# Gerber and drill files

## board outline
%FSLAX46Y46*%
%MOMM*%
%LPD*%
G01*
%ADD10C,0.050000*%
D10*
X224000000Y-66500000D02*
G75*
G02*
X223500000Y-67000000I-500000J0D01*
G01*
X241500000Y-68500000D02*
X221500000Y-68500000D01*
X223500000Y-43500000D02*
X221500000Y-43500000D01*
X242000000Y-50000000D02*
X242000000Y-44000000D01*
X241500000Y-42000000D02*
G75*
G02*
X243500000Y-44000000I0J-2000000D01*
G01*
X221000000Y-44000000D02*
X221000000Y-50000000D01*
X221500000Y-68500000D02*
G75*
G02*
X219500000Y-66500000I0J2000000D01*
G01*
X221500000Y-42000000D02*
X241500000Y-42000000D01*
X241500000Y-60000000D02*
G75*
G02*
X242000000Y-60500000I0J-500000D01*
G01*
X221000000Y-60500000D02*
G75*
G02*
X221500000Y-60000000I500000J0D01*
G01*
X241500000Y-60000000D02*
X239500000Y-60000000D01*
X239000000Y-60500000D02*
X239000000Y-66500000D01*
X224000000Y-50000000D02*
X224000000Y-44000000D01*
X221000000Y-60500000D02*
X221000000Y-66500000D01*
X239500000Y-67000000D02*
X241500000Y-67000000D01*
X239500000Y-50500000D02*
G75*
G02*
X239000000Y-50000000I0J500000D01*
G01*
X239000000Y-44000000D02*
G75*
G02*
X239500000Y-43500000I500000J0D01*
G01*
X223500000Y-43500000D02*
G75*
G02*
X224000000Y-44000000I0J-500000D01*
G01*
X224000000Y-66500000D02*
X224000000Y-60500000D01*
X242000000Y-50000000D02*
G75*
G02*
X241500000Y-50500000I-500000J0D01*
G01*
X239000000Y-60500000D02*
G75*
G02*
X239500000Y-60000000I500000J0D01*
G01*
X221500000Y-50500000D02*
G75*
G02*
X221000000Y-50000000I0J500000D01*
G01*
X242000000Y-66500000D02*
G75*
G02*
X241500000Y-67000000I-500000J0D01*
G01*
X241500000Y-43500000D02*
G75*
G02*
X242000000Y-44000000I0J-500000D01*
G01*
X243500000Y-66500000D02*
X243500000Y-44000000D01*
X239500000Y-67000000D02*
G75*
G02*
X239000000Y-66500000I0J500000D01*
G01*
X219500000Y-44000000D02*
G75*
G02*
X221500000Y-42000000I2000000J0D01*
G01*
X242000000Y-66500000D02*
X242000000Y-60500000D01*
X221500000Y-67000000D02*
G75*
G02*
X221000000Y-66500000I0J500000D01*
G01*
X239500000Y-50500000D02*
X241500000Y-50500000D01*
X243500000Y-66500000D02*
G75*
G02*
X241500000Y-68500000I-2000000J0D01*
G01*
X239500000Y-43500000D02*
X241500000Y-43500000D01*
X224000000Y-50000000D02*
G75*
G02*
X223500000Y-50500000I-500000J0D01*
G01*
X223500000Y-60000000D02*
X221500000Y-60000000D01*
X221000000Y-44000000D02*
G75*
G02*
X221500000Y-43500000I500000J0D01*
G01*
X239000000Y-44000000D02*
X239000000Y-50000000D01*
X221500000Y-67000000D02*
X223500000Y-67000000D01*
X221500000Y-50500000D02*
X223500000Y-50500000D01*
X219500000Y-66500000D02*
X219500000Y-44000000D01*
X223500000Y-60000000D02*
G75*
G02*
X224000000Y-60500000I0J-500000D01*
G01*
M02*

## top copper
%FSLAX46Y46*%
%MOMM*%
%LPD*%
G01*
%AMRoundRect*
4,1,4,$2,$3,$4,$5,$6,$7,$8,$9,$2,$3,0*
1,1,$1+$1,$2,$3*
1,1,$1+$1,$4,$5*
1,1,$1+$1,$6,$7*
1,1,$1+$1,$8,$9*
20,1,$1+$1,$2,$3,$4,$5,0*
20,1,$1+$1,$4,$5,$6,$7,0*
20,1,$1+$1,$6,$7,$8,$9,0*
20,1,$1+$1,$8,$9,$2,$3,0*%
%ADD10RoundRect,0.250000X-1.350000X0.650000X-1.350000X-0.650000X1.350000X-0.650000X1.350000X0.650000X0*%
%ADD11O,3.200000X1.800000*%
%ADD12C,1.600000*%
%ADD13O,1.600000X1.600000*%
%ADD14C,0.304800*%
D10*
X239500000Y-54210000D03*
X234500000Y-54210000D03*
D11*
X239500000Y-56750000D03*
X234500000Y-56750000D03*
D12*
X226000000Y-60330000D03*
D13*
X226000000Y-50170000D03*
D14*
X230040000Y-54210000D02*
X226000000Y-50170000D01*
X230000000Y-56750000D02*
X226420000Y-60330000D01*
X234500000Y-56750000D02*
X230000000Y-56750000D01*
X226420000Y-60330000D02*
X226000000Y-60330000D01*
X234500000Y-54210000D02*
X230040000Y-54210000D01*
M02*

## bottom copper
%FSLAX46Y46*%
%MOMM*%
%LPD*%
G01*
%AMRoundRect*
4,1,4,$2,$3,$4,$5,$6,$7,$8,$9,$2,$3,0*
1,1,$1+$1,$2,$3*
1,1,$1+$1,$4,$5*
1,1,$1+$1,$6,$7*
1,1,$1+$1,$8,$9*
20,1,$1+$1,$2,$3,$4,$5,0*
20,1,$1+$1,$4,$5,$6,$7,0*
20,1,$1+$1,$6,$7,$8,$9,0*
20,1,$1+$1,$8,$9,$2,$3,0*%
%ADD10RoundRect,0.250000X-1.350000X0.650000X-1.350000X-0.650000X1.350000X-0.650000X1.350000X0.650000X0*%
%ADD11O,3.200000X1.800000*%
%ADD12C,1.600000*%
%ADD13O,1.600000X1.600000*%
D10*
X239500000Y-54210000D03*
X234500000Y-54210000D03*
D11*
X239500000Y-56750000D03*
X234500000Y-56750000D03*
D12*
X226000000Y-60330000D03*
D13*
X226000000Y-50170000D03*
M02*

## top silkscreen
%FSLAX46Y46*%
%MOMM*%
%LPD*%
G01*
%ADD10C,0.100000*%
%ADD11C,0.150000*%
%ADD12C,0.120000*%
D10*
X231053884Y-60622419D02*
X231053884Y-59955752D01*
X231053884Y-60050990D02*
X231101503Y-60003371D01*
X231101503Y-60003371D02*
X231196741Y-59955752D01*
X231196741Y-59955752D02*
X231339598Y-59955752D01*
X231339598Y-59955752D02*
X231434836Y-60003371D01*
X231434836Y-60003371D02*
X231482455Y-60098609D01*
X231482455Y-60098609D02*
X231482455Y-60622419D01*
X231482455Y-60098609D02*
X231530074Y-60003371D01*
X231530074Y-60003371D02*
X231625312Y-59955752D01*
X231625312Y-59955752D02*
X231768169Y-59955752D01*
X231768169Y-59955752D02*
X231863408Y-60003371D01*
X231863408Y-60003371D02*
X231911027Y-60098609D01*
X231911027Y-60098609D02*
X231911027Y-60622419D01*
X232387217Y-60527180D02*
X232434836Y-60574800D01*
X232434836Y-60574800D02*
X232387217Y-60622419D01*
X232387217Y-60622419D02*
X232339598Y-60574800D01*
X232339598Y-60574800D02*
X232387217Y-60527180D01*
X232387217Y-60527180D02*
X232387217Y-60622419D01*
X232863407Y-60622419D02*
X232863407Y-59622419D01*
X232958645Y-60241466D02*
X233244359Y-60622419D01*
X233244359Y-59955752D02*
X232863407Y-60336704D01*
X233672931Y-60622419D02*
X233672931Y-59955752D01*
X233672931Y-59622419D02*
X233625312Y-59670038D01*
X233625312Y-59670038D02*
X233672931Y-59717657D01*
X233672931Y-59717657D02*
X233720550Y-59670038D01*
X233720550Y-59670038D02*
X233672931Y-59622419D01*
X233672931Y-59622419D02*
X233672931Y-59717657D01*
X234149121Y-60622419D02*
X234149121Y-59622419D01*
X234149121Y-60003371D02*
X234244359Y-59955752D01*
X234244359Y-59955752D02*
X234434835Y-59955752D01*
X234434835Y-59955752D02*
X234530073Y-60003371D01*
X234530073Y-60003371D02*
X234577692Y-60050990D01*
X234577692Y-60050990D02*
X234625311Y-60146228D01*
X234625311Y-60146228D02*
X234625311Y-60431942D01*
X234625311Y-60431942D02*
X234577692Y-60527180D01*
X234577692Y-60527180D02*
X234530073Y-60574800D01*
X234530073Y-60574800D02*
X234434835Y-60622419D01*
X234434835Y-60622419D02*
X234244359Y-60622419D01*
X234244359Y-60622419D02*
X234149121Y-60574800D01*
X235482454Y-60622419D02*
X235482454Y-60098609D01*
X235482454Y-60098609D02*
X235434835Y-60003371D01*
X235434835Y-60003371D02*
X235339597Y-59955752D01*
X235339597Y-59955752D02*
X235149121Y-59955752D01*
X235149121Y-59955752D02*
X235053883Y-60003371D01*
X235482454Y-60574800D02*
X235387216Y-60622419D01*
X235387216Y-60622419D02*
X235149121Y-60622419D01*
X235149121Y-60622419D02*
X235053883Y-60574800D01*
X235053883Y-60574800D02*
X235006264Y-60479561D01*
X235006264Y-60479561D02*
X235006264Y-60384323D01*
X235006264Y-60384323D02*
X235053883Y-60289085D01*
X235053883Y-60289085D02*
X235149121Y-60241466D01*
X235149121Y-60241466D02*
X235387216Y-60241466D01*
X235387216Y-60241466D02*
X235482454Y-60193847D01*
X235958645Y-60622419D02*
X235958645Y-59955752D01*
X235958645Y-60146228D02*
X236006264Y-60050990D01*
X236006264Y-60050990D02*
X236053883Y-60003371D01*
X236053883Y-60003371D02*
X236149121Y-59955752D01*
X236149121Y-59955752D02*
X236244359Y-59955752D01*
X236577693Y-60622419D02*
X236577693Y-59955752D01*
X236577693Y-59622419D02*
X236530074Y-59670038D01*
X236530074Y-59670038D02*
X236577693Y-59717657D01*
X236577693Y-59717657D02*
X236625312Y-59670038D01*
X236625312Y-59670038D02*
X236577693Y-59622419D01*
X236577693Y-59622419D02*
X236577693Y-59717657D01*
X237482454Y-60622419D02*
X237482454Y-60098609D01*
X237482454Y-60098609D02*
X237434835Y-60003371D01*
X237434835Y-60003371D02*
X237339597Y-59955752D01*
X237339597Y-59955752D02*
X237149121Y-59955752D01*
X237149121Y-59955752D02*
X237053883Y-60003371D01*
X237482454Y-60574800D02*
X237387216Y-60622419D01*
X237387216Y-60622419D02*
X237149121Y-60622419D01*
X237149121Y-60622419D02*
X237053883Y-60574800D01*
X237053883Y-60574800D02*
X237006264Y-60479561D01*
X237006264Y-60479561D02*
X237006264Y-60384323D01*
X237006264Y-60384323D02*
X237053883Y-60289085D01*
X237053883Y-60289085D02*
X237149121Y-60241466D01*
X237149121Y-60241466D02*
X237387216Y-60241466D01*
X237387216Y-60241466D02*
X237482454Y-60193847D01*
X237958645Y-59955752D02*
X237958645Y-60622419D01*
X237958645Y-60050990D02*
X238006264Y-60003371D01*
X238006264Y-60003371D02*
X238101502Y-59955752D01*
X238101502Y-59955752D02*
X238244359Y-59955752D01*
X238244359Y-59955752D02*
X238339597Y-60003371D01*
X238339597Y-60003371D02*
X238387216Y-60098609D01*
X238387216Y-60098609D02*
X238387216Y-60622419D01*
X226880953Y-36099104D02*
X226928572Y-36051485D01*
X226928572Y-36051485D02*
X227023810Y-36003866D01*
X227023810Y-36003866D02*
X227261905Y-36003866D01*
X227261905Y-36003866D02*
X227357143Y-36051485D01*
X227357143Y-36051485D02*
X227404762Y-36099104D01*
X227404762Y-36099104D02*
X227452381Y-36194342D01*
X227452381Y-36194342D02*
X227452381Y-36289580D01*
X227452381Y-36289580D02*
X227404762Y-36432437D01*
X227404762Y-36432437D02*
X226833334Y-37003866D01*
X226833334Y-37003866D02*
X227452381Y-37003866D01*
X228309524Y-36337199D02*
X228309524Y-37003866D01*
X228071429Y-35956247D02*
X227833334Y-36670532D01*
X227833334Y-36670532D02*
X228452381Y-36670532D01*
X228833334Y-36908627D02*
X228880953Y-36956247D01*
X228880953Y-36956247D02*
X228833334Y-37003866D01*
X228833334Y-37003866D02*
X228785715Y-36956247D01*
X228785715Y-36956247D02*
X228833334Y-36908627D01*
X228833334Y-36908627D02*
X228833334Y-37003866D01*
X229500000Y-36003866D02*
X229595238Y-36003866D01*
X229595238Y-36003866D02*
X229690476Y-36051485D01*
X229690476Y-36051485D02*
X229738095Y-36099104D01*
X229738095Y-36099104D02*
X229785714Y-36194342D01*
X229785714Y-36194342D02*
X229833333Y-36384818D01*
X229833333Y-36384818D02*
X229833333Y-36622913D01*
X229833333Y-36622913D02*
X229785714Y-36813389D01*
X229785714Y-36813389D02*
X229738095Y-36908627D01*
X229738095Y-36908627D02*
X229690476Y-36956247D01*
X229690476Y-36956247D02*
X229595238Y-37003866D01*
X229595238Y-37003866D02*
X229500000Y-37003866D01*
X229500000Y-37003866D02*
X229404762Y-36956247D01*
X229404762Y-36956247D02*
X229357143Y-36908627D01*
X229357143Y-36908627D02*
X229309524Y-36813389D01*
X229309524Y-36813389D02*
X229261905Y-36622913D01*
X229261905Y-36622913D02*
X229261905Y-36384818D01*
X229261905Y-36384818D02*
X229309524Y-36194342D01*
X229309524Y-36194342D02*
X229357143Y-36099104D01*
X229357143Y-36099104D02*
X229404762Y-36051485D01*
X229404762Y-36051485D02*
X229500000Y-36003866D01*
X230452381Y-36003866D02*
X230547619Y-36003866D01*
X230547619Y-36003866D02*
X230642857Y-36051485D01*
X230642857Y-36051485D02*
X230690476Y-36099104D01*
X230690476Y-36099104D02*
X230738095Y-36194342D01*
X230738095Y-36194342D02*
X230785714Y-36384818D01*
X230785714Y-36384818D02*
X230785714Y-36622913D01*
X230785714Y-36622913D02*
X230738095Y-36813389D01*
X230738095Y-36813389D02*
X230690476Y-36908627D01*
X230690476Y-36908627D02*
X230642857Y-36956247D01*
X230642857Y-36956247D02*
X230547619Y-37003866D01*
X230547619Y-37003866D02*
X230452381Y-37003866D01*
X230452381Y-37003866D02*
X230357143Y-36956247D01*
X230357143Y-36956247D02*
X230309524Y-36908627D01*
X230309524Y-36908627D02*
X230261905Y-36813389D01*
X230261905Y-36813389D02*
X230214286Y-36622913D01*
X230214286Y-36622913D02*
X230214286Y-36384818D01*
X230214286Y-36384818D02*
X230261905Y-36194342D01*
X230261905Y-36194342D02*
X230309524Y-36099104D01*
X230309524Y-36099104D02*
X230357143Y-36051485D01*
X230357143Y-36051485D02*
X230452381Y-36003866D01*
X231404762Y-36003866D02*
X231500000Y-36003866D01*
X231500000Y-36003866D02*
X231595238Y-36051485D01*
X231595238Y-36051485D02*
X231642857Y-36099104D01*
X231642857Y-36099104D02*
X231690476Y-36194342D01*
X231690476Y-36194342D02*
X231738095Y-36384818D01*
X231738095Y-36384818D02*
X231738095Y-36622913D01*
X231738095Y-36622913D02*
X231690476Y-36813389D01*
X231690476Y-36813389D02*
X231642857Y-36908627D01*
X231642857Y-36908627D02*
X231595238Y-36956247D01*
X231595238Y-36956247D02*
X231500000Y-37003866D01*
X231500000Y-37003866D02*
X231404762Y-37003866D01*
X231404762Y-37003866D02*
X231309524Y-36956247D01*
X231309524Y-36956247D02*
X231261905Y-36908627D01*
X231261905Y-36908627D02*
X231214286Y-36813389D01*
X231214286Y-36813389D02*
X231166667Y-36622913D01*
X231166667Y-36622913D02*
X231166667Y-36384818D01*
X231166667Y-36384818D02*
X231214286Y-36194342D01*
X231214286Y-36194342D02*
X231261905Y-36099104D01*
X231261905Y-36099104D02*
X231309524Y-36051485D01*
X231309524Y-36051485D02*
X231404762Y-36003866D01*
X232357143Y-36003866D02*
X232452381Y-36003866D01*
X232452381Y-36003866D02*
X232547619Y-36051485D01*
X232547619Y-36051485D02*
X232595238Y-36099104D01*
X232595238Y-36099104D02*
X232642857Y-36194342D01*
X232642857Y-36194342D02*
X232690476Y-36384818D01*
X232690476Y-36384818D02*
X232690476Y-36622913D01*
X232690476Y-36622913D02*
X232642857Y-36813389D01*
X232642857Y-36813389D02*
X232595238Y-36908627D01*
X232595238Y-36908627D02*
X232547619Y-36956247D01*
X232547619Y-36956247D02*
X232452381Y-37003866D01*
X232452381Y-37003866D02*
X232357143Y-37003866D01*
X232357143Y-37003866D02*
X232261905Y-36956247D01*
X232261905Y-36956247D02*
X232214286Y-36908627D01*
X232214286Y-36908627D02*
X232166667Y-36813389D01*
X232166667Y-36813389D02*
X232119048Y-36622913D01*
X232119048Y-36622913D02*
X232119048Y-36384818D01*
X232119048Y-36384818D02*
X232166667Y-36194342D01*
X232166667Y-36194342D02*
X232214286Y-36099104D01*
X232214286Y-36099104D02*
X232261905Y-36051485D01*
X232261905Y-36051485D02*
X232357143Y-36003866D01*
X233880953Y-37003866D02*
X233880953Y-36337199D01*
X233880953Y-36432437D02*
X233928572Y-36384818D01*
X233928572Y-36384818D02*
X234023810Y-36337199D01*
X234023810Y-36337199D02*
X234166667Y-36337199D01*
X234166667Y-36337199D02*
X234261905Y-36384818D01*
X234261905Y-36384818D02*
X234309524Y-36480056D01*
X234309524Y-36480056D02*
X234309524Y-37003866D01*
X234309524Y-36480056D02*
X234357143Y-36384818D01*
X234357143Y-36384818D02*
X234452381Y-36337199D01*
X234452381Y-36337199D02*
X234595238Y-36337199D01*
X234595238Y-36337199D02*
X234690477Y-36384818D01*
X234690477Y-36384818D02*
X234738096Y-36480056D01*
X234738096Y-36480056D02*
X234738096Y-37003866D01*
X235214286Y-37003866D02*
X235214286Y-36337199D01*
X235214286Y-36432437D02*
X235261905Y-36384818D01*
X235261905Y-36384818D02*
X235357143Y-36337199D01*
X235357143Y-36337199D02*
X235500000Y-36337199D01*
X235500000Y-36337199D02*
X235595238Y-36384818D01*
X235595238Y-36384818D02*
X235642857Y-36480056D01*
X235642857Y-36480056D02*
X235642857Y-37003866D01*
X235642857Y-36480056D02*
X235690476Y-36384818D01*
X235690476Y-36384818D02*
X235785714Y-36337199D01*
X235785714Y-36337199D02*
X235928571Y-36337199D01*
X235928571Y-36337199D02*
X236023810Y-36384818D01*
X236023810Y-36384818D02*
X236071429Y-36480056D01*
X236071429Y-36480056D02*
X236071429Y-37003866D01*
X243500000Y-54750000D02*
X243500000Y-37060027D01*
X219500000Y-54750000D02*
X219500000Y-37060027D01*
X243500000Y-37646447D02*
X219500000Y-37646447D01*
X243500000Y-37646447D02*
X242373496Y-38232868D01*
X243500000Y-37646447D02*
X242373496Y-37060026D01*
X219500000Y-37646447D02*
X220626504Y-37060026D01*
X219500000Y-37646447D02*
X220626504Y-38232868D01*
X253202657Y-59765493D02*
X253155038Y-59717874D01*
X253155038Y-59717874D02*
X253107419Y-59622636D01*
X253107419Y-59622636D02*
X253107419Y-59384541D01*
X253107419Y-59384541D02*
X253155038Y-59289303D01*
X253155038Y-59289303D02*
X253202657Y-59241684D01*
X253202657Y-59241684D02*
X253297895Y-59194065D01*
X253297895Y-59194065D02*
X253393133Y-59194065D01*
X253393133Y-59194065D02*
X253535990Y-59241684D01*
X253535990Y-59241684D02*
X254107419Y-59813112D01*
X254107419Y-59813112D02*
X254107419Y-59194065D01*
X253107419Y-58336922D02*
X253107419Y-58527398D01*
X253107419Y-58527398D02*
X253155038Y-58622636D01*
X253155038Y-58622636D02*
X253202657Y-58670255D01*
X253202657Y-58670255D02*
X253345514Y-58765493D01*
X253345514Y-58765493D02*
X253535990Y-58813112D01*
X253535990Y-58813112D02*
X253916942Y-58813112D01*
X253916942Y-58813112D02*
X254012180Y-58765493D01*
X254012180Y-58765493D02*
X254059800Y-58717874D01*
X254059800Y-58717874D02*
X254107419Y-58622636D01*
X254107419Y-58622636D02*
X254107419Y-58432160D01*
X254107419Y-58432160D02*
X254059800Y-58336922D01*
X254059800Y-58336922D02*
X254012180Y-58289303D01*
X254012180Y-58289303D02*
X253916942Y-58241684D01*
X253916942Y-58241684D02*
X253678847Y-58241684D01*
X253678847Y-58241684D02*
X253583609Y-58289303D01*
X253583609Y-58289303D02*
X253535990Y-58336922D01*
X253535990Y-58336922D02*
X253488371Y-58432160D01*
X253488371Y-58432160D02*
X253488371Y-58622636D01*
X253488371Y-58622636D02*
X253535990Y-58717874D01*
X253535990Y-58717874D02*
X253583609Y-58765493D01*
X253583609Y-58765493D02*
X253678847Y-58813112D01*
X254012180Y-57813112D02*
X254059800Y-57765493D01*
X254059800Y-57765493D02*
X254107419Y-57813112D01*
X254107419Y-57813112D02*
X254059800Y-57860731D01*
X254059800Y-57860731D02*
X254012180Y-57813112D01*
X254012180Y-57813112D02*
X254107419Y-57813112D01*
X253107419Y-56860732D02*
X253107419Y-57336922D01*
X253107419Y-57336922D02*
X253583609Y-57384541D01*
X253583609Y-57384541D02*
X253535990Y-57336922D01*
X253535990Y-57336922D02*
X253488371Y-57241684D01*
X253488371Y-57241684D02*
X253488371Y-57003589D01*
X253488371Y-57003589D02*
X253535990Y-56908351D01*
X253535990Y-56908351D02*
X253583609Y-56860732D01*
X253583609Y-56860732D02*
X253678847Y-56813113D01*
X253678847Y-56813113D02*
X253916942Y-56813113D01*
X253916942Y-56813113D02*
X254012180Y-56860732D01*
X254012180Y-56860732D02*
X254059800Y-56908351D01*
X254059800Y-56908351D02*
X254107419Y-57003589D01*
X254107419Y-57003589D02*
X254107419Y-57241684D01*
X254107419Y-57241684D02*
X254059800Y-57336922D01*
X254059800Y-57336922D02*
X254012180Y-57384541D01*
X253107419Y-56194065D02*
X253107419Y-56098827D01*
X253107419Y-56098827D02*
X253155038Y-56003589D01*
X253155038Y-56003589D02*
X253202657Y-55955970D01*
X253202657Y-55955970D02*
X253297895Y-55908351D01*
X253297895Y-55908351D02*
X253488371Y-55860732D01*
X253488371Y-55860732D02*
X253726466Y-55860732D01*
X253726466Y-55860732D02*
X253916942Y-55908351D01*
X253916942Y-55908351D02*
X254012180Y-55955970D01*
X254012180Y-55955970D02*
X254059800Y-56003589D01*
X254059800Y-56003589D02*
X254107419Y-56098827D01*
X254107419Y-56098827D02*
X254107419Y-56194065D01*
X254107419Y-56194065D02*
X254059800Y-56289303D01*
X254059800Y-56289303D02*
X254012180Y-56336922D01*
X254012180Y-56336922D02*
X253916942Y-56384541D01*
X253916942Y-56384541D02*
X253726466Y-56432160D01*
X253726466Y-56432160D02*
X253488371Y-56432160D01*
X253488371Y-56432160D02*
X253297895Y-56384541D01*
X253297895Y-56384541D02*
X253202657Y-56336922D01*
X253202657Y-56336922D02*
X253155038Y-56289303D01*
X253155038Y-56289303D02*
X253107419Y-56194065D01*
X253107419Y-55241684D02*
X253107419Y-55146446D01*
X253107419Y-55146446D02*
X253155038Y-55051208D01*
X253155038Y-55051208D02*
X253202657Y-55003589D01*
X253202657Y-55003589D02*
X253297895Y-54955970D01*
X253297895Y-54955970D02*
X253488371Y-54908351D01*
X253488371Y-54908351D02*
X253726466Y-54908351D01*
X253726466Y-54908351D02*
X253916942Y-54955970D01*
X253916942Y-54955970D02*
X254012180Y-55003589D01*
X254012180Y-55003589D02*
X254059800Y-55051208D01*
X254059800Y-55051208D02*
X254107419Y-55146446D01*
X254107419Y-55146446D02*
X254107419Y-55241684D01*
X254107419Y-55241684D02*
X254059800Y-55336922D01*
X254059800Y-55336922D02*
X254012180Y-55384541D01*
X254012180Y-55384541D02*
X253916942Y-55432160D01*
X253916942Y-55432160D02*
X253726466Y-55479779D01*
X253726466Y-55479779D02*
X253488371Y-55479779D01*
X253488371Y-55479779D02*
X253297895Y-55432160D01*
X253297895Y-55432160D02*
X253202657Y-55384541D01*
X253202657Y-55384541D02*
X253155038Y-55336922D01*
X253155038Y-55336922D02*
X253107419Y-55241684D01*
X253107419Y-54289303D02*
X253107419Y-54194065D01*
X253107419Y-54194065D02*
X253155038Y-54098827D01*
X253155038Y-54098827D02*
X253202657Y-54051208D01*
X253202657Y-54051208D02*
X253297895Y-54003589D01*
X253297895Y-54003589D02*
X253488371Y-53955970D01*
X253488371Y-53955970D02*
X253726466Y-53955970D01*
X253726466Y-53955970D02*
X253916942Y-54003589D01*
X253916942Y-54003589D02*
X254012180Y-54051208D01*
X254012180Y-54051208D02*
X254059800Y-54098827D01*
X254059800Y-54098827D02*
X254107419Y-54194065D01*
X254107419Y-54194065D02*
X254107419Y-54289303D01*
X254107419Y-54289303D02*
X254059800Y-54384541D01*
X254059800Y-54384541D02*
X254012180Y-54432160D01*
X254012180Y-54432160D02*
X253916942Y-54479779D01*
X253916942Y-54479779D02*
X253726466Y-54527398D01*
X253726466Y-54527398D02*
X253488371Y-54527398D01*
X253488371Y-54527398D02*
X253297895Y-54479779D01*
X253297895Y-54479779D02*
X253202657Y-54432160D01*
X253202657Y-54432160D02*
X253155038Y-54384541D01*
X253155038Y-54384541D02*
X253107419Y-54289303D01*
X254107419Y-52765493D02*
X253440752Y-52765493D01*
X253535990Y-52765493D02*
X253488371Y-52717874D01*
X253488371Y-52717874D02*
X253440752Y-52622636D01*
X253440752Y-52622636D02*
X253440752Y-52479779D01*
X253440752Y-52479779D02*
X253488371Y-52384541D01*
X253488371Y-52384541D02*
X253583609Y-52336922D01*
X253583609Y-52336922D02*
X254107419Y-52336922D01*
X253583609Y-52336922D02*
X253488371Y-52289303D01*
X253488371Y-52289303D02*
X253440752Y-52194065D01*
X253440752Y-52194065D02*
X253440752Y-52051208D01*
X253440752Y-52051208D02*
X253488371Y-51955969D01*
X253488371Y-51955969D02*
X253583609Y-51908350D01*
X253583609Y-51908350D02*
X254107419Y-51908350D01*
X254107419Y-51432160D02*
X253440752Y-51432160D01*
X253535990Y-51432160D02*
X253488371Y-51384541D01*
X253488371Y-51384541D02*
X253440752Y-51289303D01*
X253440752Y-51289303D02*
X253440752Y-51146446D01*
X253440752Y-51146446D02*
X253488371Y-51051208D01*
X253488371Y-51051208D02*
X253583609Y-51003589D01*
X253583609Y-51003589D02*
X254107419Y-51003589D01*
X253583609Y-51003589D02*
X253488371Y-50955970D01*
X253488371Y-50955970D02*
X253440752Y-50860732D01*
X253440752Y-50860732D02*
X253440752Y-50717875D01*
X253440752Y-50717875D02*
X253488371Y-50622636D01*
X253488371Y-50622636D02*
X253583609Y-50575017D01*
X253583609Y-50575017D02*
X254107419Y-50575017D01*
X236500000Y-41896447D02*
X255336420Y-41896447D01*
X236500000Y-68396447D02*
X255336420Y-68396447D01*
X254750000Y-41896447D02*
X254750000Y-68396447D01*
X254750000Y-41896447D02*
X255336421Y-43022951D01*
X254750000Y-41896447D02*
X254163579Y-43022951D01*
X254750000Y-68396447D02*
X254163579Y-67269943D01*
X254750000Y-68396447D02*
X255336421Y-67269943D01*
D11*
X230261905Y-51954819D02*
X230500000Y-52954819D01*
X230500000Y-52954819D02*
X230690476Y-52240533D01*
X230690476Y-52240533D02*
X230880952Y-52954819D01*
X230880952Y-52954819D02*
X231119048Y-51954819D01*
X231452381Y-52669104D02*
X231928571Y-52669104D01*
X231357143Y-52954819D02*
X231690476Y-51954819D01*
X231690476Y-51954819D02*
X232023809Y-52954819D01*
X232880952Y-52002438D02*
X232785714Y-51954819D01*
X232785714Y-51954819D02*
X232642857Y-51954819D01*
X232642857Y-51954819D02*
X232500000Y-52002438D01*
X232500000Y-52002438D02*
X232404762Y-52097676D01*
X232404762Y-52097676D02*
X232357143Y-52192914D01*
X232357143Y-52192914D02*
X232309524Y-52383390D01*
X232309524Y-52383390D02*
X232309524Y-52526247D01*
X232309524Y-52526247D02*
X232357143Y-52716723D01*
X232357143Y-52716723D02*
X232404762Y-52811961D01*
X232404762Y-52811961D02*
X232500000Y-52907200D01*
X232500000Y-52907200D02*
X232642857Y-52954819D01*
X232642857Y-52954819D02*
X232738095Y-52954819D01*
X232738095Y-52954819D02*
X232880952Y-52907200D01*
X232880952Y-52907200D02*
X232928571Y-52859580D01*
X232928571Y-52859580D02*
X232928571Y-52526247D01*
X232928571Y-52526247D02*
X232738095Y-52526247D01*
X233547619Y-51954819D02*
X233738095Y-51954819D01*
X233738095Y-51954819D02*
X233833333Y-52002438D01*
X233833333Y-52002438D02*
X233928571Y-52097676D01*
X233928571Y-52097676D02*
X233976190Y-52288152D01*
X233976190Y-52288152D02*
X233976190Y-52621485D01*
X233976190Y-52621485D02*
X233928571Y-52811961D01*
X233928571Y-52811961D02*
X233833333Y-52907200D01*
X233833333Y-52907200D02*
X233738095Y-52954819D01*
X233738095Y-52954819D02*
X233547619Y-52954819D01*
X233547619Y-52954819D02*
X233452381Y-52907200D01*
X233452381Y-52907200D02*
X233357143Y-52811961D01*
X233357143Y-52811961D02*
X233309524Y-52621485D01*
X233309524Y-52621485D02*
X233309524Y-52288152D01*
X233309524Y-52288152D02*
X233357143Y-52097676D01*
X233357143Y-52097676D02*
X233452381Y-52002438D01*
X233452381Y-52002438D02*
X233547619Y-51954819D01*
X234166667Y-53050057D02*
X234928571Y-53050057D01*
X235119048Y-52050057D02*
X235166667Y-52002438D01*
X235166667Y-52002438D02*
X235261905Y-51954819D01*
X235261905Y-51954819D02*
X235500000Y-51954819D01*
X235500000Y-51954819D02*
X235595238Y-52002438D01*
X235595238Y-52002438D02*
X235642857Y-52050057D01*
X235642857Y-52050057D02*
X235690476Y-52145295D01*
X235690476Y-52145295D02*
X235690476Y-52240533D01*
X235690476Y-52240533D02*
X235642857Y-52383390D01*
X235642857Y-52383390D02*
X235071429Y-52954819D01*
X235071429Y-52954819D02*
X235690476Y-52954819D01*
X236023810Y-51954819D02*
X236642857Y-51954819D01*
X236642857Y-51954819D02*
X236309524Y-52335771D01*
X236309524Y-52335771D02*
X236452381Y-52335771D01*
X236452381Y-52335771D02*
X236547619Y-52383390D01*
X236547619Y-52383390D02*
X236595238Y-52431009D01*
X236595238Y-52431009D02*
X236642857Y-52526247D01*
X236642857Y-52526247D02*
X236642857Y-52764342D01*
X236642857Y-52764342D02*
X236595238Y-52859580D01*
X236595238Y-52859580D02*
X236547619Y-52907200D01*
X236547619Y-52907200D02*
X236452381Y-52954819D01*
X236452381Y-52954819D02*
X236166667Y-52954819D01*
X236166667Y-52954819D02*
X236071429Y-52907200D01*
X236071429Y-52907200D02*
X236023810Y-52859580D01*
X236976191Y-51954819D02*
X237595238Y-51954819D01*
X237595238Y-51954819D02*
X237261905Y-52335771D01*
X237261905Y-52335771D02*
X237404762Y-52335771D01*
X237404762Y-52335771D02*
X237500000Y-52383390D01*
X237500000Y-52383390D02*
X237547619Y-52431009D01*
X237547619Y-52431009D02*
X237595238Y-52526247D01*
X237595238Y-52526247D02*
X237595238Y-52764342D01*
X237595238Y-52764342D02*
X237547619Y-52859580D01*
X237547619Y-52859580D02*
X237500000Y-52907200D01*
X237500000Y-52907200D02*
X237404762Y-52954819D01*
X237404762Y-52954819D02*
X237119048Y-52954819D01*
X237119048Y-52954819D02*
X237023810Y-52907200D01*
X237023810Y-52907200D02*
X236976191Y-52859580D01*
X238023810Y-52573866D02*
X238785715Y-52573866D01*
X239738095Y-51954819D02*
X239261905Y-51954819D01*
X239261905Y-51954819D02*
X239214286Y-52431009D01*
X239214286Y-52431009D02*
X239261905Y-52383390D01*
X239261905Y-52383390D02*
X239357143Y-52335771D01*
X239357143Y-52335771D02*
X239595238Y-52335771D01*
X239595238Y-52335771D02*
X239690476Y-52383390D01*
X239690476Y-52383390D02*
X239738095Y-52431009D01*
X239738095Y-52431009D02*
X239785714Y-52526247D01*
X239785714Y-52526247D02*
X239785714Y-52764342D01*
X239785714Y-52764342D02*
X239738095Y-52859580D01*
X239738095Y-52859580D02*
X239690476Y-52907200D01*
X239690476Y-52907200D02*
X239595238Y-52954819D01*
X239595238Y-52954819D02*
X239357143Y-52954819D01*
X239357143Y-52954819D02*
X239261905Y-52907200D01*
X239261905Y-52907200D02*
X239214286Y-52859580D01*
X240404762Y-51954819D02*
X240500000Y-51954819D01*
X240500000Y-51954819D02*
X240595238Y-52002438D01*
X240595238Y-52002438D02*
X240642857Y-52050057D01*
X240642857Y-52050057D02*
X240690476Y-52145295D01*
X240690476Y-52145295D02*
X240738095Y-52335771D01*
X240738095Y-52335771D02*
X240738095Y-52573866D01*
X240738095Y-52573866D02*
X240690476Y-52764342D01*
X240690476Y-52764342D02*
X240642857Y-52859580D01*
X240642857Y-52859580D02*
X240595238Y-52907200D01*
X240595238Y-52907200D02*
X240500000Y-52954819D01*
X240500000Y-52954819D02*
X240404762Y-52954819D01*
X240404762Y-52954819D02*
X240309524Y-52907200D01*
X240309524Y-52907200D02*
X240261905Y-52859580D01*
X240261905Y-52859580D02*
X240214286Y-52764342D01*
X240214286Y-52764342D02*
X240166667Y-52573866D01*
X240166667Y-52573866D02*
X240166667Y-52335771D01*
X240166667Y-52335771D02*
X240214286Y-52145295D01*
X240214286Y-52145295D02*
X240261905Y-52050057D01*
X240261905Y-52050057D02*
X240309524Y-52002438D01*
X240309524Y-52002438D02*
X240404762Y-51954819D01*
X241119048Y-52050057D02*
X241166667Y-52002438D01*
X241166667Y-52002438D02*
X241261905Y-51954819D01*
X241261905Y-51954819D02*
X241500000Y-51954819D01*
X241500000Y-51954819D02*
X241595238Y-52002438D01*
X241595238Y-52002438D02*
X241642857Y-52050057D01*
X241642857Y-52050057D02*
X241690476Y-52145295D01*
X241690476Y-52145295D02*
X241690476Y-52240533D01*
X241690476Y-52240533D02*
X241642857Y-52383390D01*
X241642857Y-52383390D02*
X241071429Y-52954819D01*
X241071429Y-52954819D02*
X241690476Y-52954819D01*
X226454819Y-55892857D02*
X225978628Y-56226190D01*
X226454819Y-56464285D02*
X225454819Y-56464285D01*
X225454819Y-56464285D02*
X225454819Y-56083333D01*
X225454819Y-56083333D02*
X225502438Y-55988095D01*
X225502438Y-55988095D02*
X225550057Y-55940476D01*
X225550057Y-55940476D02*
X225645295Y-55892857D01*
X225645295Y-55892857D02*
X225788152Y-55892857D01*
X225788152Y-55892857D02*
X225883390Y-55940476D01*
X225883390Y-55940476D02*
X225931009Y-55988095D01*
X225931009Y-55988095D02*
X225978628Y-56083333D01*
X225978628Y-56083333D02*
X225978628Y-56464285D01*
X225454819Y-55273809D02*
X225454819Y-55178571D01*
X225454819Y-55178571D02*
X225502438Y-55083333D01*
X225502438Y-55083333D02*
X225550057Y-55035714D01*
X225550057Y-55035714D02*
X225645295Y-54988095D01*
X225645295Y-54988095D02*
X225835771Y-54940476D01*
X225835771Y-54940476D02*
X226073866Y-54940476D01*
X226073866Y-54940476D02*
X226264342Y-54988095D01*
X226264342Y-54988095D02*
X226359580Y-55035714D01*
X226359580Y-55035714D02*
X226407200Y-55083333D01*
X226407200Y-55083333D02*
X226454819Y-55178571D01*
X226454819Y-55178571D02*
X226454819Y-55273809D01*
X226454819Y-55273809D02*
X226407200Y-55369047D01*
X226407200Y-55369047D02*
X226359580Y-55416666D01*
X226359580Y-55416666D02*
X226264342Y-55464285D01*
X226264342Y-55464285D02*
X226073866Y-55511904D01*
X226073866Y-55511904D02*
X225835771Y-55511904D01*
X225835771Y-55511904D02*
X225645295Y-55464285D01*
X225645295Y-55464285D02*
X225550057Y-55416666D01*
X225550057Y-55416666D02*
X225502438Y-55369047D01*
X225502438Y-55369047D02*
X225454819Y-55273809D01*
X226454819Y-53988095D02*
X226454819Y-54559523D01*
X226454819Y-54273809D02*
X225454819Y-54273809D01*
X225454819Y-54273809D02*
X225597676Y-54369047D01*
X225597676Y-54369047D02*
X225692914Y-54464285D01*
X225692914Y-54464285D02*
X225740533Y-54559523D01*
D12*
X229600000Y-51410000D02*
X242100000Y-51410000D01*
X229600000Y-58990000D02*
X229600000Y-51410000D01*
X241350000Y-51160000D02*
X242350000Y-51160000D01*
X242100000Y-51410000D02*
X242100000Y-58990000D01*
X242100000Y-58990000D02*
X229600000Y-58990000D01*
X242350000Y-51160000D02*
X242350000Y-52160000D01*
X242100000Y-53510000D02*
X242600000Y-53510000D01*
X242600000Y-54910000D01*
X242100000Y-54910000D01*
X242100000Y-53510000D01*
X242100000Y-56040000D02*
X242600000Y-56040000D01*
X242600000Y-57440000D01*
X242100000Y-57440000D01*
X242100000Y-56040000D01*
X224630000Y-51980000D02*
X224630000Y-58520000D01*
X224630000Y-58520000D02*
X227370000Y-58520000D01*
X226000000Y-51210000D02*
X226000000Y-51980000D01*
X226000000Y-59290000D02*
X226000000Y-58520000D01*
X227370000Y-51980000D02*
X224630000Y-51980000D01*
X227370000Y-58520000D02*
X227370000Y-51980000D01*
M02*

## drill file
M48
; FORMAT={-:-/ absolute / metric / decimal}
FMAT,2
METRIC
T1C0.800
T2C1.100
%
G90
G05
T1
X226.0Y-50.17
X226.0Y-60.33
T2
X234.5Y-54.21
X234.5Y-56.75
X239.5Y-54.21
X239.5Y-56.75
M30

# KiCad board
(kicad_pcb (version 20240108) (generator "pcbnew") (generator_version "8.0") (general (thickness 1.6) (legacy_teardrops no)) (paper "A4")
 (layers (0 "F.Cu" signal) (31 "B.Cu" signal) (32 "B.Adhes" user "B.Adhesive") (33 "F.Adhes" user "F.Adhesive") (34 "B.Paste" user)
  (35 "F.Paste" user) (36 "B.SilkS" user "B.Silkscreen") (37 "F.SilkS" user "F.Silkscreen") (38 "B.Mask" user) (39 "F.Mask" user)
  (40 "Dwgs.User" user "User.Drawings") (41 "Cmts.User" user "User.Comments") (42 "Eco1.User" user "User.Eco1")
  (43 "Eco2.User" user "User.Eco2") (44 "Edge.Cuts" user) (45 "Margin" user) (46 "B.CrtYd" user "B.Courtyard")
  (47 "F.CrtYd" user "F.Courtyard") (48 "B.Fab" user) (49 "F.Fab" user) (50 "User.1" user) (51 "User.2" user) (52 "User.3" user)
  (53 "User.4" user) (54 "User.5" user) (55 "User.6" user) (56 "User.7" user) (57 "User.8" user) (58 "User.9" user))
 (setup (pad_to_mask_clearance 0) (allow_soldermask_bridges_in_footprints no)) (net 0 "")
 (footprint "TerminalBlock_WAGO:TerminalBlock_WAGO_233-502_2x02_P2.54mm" (layer "F.Cu") (at 239.5 54.21 -90)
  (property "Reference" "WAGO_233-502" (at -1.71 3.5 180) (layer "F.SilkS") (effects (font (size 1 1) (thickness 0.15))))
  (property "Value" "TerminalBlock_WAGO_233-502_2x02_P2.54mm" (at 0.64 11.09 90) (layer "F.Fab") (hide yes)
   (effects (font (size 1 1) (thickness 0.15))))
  (fp_line (start -2.8 9.9) (end -2.8 -2.6) (stroke (width 0.12) (type solid)) (layer "F.SilkS"))
  (fp_line (start 4.78 9.9) (end -2.8 9.9) (stroke (width 0.12) (type solid)) (layer "F.SilkS"))
  (fp_line (start -3.05 -1.85) (end -3.05 -2.85) (stroke (width 0.12) (type default)) (layer "F.SilkS"))
  (fp_line (start -2.8 -2.6) (end 4.78 -2.6) (stroke (width 0.12) (type solid)) (layer "F.SilkS"))
  (fp_line (start 4.78 -2.6) (end 4.78 9.9) (stroke (width 0.12) (type solid)) (layer "F.SilkS"))
  (fp_line (start -3.05 -2.85) (end -2.05 -2.85) (stroke (width 0.12) (type default)) (layer "F.SilkS"))
  (fp_rect (start -0.7 -3.1) (end 0.7 -2.6) (stroke (width 0.12) (type default)) (fill none) (layer "F.SilkS"))
  (fp_rect (start 1.83 -3.1) (end 3.23 -2.6) (stroke (width 0.12) (type default)) (fill none) (layer "F.SilkS"))
  (pad "1" thru_hole roundrect (at 0 0 270) (size 1.8 3.2) (drill 1.1) (layers "*.Cu" "*.Mask") (remove_unused_layers no)
   (roundrect_rratio 0.1388888889))
  (pad "1" thru_hole roundrect (at 0 5 270) (size 1.8 3.2) (drill 1.1) (layers "*.Cu" "*.Mask") (remove_unused_layers no)
   (roundrect_rratio 0.1388888889))
  (pad "2" thru_hole oval (at 2.54 0 270) (size 1.8 3.2) (drill 1.1) (layers "*.Cu" "*.Mask") (remove_unused_layers no))
  (pad "2" thru_hole oval (at 2.54 5 270) (size 1.8 3.2) (drill 1.1) (layers "*.Cu" "*.Mask") (remove_unused_layers no)))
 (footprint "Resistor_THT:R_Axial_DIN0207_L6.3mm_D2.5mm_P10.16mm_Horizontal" (layer "F.Cu") (at 226 60.33 90)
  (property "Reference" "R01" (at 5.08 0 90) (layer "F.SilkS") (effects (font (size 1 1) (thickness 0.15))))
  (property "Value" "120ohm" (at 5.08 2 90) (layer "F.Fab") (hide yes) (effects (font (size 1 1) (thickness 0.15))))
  (fp_line (start 8.35 -1.37) (end 1.81 -1.37) (stroke (width 0.12) (type solid)) (layer "F.SilkS"))
  (fp_line (start 1.81 -1.37) (end 1.81 1.37) (stroke (width 0.12) (type solid)) (layer "F.SilkS"))
  (fp_line (start 9.12 0) (end 8.35 0) (stroke (width 0.12) (type solid)) (layer "F.SilkS"))
  (fp_line (start 1.04 0) (end 1.81 0) (stroke (width 0.12) (type solid)) (layer "F.SilkS"))
  (fp_line (start 8.35 1.37) (end 8.35 -1.37) (stroke (width 0.12) (type solid)) (layer "F.SilkS"))
  (fp_line (start 1.81 1.37) (end 8.35 1.37) (stroke (width 0.12) (type solid)) (layer "F.SilkS"))
  (pad "1" thru_hole circle (at 0 0 90) (size 1.6 1.6) (drill 0.8) (layers "*.Cu" "*.Mask") (remove_unused_layers no))
  (pad "2" thru_hole oval (at 10.16 0 90) (size 1.6 1.6) (drill 0.8) (layers "*.Cu" "*.Mask") (remove_unused_layers no)))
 (gr_arc (start 224 66.5) (mid 223.853553 66.853553) (end 223.5 67) (stroke (width 0.05) (type default)) (layer "Edge.Cuts"))
 (gr_line (start 241.5 68.5) (end 221.5 68.5) (stroke (width 0.05) (type default)) (layer "Edge.Cuts"))
 (gr_line (start 223.5 43.5) (end 221.5 43.5) (stroke (width 0.05) (type default)) (layer "Edge.Cuts"))
 (gr_line (start 242 50) (end 242 44) (stroke (width 0.05) (type default)) (layer "Edge.Cuts"))
 (gr_arc (start 241.5 42) (mid 242.914214 42.585786) (end 243.5 44) (stroke (width 0.05) (type default)) (layer "Edge.Cuts"))
 (gr_line (start 221 44) (end 221 50) (stroke (width 0.05) (type default)) (layer "Edge.Cuts"))
 (gr_arc (start 221.5 68.5) (mid 220.085786 67.914214) (end 219.5 66.5) (stroke (width 0.05) (type default)) (layer "Edge.Cuts"))
 (gr_line (start 221.5 42) (end 241.5 42) (stroke (width 0.05) (type default)) (layer "Edge.Cuts"))
 (gr_arc (start 241.5 60) (mid 241.853553 60.146447) (end 242 60.5) (stroke (width 0.05) (type default)) (layer "Edge.Cuts"))
 (gr_arc (start 221 60.5) (mid 221.146447 60.146447) (end 221.5 60) (stroke (width 0.05) (type default)) (layer "Edge.Cuts"))
 (gr_line (start 241.5 60) (end 239.5 60) (stroke (width 0.05) (type default)) (layer "Edge.Cuts"))
 (gr_line (start 239 60.5) (end 239 66.5) (stroke (width 0.05) (type default)) (layer "Edge.Cuts"))
 (gr_line (start 224 50) (end 224 44) (stroke (width 0.05) (type default)) (layer "Edge.Cuts"))
 (gr_line (start 221 60.5) (end 221 66.5) (stroke (width 0.05) (type default)) (layer "Edge.Cuts"))
 (gr_line (start 239.5 67) (end 241.5 67) (stroke (width 0.05) (type default)) (layer "Edge.Cuts"))
 (gr_arc (start 239.5 50.5) (mid 239.146447 50.353553) (end 239 50) (stroke (width 0.05) (type default)) (layer "Edge.Cuts"))
 (gr_arc (start 239 44) (mid 239.146447 43.646447) (end 239.5 43.5) (stroke (width 0.05) (type default)) (layer "Edge.Cuts"))
 (gr_arc (start 223.5 43.5) (mid 223.853553 43.646447) (end 224 44) (stroke (width 0.05) (type default)) (layer "Edge.Cuts"))
 (gr_line (start 224 66.5) (end 224 60.5) (stroke (width 0.05) (type default)) (layer "Edge.Cuts"))
 (gr_arc (start 242 50) (mid 241.853553 50.353553) (end 241.5 50.5) (stroke (width 0.05) (type default)) (layer "Edge.Cuts"))
 (gr_arc (start 239 60.5) (mid 239.146447 60.146447) (end 239.5 60) (stroke (width 0.05) (type default)) (layer "Edge.Cuts"))
 (gr_arc (start 221.5 50.5) (mid 221.146447 50.353553) (end 221 50) (stroke (width 0.05) (type default)) (layer "Edge.Cuts"))
 (gr_arc (start 242 66.5) (mid 241.853553 66.853553) (end 241.5 67) (stroke (width 0.05) (type default)) (layer "Edge.Cuts"))
 (gr_arc (start 241.5 43.5) (mid 241.853553 43.646447) (end 242 44) (stroke (width 0.05) (type default)) (layer "Edge.Cuts"))
 (gr_line (start 243.5 66.5) (end 243.5 44) (stroke (width 0.05) (type default)) (layer "Edge.Cuts"))
 (gr_arc (start 239.5 67) (mid 239.146447 66.853553) (end 239 66.5) (stroke (width 0.05) (type default)) (layer "Edge.Cuts"))
 (gr_arc (start 219.5 44) (mid 220.085786 42.585786) (end 221.5 42) (stroke (width 0.05) (type default)) (layer "Edge.Cuts"))
 (gr_line (start 242 66.5) (end 242 60.5) (stroke (width 0.05) (type default)) (layer "Edge.Cuts"))
 (gr_arc (start 221.5 67) (mid 221.146447 66.853553) (end 221 66.5) (stroke (width 0.05) (type default)) (layer "Edge.Cuts"))
 (gr_line (start 239.5 50.5) (end 241.5 50.5) (stroke (width 0.05) (type default)) (layer "Edge.Cuts"))
 (gr_arc (start 243.5 66.5) (mid 242.914214 67.914214) (end 241.5 68.5) (stroke (width 0.05) (type default)) (layer "Edge.Cuts"))
 (gr_line (start 239.5 43.5) (end 241.5 43.5) (stroke (width 0.05) (type default)) (layer "Edge.Cuts"))
 (gr_arc (start 224 50) (mid 223.853553 50.353553) (end 223.5 50.5) (stroke (width 0.05) (type default)) (layer "Edge.Cuts"))
 (gr_line (start 223.5 60) (end 221.5 60) (stroke (width 0.05) (type default)) (layer "Edge.Cuts"))
 (gr_arc (start 221 44) (mid 221.146447 43.646447) (end 221.5 43.5) (stroke (width 0.05) (type default)) (layer "Edge.Cuts"))
 (gr_line (start 239 44) (end 239 50) (stroke (width 0.05) (type default)) (layer "Edge.Cuts"))
 (gr_line (start 221.5 67) (end 223.5 67) (stroke (width 0.05) (type default)) (layer "Edge.Cuts"))
 (gr_line (start 221.5 50.5) (end 223.5 50.5) (stroke (width 0.05) (type default)) (layer "Edge.Cuts"))
 (gr_line (start 219.5 66.5) (end 219.5 44) (stroke (width 0.05) (type default)) (layer "Edge.Cuts"))
 (gr_arc (start 223.5 60) (mid 223.853553 60.146447) (end 224 60.5) (stroke (width 0.05) (type default)) (layer "Edge.Cuts"))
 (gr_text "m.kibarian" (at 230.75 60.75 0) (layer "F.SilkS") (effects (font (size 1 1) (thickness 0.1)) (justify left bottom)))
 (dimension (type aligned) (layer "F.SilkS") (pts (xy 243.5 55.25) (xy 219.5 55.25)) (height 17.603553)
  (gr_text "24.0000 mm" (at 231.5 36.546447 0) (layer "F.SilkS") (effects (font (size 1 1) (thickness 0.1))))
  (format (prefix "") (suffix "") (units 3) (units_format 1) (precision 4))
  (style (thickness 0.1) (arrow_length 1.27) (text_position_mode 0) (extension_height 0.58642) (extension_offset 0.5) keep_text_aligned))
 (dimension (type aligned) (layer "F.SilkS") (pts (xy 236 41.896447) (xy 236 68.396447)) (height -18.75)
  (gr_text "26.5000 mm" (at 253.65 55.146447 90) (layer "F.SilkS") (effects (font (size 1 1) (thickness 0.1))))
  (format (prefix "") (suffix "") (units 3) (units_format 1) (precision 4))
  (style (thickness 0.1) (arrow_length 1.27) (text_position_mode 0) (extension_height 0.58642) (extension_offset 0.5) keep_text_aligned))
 (segment (start 230.04 54.21) (end 226 50.17) (width 0.3048) (layer "F.Cu") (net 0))
 (segment (start 230 56.75) (end 226.42 60.33) (width 0.3048) (layer "F.Cu") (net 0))
 (segment (start 234.5 56.75) (end 230 56.75) (width 0.3048) (layer "F.Cu") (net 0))
 (segment (start 226.42 60.33) (end 226 60.33) (width 0.3048) (layer "F.Cu") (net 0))
 (segment (start 234.5 54.21) (end 230.04 54.21) (width 0.3048) (layer "F.Cu") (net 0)))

